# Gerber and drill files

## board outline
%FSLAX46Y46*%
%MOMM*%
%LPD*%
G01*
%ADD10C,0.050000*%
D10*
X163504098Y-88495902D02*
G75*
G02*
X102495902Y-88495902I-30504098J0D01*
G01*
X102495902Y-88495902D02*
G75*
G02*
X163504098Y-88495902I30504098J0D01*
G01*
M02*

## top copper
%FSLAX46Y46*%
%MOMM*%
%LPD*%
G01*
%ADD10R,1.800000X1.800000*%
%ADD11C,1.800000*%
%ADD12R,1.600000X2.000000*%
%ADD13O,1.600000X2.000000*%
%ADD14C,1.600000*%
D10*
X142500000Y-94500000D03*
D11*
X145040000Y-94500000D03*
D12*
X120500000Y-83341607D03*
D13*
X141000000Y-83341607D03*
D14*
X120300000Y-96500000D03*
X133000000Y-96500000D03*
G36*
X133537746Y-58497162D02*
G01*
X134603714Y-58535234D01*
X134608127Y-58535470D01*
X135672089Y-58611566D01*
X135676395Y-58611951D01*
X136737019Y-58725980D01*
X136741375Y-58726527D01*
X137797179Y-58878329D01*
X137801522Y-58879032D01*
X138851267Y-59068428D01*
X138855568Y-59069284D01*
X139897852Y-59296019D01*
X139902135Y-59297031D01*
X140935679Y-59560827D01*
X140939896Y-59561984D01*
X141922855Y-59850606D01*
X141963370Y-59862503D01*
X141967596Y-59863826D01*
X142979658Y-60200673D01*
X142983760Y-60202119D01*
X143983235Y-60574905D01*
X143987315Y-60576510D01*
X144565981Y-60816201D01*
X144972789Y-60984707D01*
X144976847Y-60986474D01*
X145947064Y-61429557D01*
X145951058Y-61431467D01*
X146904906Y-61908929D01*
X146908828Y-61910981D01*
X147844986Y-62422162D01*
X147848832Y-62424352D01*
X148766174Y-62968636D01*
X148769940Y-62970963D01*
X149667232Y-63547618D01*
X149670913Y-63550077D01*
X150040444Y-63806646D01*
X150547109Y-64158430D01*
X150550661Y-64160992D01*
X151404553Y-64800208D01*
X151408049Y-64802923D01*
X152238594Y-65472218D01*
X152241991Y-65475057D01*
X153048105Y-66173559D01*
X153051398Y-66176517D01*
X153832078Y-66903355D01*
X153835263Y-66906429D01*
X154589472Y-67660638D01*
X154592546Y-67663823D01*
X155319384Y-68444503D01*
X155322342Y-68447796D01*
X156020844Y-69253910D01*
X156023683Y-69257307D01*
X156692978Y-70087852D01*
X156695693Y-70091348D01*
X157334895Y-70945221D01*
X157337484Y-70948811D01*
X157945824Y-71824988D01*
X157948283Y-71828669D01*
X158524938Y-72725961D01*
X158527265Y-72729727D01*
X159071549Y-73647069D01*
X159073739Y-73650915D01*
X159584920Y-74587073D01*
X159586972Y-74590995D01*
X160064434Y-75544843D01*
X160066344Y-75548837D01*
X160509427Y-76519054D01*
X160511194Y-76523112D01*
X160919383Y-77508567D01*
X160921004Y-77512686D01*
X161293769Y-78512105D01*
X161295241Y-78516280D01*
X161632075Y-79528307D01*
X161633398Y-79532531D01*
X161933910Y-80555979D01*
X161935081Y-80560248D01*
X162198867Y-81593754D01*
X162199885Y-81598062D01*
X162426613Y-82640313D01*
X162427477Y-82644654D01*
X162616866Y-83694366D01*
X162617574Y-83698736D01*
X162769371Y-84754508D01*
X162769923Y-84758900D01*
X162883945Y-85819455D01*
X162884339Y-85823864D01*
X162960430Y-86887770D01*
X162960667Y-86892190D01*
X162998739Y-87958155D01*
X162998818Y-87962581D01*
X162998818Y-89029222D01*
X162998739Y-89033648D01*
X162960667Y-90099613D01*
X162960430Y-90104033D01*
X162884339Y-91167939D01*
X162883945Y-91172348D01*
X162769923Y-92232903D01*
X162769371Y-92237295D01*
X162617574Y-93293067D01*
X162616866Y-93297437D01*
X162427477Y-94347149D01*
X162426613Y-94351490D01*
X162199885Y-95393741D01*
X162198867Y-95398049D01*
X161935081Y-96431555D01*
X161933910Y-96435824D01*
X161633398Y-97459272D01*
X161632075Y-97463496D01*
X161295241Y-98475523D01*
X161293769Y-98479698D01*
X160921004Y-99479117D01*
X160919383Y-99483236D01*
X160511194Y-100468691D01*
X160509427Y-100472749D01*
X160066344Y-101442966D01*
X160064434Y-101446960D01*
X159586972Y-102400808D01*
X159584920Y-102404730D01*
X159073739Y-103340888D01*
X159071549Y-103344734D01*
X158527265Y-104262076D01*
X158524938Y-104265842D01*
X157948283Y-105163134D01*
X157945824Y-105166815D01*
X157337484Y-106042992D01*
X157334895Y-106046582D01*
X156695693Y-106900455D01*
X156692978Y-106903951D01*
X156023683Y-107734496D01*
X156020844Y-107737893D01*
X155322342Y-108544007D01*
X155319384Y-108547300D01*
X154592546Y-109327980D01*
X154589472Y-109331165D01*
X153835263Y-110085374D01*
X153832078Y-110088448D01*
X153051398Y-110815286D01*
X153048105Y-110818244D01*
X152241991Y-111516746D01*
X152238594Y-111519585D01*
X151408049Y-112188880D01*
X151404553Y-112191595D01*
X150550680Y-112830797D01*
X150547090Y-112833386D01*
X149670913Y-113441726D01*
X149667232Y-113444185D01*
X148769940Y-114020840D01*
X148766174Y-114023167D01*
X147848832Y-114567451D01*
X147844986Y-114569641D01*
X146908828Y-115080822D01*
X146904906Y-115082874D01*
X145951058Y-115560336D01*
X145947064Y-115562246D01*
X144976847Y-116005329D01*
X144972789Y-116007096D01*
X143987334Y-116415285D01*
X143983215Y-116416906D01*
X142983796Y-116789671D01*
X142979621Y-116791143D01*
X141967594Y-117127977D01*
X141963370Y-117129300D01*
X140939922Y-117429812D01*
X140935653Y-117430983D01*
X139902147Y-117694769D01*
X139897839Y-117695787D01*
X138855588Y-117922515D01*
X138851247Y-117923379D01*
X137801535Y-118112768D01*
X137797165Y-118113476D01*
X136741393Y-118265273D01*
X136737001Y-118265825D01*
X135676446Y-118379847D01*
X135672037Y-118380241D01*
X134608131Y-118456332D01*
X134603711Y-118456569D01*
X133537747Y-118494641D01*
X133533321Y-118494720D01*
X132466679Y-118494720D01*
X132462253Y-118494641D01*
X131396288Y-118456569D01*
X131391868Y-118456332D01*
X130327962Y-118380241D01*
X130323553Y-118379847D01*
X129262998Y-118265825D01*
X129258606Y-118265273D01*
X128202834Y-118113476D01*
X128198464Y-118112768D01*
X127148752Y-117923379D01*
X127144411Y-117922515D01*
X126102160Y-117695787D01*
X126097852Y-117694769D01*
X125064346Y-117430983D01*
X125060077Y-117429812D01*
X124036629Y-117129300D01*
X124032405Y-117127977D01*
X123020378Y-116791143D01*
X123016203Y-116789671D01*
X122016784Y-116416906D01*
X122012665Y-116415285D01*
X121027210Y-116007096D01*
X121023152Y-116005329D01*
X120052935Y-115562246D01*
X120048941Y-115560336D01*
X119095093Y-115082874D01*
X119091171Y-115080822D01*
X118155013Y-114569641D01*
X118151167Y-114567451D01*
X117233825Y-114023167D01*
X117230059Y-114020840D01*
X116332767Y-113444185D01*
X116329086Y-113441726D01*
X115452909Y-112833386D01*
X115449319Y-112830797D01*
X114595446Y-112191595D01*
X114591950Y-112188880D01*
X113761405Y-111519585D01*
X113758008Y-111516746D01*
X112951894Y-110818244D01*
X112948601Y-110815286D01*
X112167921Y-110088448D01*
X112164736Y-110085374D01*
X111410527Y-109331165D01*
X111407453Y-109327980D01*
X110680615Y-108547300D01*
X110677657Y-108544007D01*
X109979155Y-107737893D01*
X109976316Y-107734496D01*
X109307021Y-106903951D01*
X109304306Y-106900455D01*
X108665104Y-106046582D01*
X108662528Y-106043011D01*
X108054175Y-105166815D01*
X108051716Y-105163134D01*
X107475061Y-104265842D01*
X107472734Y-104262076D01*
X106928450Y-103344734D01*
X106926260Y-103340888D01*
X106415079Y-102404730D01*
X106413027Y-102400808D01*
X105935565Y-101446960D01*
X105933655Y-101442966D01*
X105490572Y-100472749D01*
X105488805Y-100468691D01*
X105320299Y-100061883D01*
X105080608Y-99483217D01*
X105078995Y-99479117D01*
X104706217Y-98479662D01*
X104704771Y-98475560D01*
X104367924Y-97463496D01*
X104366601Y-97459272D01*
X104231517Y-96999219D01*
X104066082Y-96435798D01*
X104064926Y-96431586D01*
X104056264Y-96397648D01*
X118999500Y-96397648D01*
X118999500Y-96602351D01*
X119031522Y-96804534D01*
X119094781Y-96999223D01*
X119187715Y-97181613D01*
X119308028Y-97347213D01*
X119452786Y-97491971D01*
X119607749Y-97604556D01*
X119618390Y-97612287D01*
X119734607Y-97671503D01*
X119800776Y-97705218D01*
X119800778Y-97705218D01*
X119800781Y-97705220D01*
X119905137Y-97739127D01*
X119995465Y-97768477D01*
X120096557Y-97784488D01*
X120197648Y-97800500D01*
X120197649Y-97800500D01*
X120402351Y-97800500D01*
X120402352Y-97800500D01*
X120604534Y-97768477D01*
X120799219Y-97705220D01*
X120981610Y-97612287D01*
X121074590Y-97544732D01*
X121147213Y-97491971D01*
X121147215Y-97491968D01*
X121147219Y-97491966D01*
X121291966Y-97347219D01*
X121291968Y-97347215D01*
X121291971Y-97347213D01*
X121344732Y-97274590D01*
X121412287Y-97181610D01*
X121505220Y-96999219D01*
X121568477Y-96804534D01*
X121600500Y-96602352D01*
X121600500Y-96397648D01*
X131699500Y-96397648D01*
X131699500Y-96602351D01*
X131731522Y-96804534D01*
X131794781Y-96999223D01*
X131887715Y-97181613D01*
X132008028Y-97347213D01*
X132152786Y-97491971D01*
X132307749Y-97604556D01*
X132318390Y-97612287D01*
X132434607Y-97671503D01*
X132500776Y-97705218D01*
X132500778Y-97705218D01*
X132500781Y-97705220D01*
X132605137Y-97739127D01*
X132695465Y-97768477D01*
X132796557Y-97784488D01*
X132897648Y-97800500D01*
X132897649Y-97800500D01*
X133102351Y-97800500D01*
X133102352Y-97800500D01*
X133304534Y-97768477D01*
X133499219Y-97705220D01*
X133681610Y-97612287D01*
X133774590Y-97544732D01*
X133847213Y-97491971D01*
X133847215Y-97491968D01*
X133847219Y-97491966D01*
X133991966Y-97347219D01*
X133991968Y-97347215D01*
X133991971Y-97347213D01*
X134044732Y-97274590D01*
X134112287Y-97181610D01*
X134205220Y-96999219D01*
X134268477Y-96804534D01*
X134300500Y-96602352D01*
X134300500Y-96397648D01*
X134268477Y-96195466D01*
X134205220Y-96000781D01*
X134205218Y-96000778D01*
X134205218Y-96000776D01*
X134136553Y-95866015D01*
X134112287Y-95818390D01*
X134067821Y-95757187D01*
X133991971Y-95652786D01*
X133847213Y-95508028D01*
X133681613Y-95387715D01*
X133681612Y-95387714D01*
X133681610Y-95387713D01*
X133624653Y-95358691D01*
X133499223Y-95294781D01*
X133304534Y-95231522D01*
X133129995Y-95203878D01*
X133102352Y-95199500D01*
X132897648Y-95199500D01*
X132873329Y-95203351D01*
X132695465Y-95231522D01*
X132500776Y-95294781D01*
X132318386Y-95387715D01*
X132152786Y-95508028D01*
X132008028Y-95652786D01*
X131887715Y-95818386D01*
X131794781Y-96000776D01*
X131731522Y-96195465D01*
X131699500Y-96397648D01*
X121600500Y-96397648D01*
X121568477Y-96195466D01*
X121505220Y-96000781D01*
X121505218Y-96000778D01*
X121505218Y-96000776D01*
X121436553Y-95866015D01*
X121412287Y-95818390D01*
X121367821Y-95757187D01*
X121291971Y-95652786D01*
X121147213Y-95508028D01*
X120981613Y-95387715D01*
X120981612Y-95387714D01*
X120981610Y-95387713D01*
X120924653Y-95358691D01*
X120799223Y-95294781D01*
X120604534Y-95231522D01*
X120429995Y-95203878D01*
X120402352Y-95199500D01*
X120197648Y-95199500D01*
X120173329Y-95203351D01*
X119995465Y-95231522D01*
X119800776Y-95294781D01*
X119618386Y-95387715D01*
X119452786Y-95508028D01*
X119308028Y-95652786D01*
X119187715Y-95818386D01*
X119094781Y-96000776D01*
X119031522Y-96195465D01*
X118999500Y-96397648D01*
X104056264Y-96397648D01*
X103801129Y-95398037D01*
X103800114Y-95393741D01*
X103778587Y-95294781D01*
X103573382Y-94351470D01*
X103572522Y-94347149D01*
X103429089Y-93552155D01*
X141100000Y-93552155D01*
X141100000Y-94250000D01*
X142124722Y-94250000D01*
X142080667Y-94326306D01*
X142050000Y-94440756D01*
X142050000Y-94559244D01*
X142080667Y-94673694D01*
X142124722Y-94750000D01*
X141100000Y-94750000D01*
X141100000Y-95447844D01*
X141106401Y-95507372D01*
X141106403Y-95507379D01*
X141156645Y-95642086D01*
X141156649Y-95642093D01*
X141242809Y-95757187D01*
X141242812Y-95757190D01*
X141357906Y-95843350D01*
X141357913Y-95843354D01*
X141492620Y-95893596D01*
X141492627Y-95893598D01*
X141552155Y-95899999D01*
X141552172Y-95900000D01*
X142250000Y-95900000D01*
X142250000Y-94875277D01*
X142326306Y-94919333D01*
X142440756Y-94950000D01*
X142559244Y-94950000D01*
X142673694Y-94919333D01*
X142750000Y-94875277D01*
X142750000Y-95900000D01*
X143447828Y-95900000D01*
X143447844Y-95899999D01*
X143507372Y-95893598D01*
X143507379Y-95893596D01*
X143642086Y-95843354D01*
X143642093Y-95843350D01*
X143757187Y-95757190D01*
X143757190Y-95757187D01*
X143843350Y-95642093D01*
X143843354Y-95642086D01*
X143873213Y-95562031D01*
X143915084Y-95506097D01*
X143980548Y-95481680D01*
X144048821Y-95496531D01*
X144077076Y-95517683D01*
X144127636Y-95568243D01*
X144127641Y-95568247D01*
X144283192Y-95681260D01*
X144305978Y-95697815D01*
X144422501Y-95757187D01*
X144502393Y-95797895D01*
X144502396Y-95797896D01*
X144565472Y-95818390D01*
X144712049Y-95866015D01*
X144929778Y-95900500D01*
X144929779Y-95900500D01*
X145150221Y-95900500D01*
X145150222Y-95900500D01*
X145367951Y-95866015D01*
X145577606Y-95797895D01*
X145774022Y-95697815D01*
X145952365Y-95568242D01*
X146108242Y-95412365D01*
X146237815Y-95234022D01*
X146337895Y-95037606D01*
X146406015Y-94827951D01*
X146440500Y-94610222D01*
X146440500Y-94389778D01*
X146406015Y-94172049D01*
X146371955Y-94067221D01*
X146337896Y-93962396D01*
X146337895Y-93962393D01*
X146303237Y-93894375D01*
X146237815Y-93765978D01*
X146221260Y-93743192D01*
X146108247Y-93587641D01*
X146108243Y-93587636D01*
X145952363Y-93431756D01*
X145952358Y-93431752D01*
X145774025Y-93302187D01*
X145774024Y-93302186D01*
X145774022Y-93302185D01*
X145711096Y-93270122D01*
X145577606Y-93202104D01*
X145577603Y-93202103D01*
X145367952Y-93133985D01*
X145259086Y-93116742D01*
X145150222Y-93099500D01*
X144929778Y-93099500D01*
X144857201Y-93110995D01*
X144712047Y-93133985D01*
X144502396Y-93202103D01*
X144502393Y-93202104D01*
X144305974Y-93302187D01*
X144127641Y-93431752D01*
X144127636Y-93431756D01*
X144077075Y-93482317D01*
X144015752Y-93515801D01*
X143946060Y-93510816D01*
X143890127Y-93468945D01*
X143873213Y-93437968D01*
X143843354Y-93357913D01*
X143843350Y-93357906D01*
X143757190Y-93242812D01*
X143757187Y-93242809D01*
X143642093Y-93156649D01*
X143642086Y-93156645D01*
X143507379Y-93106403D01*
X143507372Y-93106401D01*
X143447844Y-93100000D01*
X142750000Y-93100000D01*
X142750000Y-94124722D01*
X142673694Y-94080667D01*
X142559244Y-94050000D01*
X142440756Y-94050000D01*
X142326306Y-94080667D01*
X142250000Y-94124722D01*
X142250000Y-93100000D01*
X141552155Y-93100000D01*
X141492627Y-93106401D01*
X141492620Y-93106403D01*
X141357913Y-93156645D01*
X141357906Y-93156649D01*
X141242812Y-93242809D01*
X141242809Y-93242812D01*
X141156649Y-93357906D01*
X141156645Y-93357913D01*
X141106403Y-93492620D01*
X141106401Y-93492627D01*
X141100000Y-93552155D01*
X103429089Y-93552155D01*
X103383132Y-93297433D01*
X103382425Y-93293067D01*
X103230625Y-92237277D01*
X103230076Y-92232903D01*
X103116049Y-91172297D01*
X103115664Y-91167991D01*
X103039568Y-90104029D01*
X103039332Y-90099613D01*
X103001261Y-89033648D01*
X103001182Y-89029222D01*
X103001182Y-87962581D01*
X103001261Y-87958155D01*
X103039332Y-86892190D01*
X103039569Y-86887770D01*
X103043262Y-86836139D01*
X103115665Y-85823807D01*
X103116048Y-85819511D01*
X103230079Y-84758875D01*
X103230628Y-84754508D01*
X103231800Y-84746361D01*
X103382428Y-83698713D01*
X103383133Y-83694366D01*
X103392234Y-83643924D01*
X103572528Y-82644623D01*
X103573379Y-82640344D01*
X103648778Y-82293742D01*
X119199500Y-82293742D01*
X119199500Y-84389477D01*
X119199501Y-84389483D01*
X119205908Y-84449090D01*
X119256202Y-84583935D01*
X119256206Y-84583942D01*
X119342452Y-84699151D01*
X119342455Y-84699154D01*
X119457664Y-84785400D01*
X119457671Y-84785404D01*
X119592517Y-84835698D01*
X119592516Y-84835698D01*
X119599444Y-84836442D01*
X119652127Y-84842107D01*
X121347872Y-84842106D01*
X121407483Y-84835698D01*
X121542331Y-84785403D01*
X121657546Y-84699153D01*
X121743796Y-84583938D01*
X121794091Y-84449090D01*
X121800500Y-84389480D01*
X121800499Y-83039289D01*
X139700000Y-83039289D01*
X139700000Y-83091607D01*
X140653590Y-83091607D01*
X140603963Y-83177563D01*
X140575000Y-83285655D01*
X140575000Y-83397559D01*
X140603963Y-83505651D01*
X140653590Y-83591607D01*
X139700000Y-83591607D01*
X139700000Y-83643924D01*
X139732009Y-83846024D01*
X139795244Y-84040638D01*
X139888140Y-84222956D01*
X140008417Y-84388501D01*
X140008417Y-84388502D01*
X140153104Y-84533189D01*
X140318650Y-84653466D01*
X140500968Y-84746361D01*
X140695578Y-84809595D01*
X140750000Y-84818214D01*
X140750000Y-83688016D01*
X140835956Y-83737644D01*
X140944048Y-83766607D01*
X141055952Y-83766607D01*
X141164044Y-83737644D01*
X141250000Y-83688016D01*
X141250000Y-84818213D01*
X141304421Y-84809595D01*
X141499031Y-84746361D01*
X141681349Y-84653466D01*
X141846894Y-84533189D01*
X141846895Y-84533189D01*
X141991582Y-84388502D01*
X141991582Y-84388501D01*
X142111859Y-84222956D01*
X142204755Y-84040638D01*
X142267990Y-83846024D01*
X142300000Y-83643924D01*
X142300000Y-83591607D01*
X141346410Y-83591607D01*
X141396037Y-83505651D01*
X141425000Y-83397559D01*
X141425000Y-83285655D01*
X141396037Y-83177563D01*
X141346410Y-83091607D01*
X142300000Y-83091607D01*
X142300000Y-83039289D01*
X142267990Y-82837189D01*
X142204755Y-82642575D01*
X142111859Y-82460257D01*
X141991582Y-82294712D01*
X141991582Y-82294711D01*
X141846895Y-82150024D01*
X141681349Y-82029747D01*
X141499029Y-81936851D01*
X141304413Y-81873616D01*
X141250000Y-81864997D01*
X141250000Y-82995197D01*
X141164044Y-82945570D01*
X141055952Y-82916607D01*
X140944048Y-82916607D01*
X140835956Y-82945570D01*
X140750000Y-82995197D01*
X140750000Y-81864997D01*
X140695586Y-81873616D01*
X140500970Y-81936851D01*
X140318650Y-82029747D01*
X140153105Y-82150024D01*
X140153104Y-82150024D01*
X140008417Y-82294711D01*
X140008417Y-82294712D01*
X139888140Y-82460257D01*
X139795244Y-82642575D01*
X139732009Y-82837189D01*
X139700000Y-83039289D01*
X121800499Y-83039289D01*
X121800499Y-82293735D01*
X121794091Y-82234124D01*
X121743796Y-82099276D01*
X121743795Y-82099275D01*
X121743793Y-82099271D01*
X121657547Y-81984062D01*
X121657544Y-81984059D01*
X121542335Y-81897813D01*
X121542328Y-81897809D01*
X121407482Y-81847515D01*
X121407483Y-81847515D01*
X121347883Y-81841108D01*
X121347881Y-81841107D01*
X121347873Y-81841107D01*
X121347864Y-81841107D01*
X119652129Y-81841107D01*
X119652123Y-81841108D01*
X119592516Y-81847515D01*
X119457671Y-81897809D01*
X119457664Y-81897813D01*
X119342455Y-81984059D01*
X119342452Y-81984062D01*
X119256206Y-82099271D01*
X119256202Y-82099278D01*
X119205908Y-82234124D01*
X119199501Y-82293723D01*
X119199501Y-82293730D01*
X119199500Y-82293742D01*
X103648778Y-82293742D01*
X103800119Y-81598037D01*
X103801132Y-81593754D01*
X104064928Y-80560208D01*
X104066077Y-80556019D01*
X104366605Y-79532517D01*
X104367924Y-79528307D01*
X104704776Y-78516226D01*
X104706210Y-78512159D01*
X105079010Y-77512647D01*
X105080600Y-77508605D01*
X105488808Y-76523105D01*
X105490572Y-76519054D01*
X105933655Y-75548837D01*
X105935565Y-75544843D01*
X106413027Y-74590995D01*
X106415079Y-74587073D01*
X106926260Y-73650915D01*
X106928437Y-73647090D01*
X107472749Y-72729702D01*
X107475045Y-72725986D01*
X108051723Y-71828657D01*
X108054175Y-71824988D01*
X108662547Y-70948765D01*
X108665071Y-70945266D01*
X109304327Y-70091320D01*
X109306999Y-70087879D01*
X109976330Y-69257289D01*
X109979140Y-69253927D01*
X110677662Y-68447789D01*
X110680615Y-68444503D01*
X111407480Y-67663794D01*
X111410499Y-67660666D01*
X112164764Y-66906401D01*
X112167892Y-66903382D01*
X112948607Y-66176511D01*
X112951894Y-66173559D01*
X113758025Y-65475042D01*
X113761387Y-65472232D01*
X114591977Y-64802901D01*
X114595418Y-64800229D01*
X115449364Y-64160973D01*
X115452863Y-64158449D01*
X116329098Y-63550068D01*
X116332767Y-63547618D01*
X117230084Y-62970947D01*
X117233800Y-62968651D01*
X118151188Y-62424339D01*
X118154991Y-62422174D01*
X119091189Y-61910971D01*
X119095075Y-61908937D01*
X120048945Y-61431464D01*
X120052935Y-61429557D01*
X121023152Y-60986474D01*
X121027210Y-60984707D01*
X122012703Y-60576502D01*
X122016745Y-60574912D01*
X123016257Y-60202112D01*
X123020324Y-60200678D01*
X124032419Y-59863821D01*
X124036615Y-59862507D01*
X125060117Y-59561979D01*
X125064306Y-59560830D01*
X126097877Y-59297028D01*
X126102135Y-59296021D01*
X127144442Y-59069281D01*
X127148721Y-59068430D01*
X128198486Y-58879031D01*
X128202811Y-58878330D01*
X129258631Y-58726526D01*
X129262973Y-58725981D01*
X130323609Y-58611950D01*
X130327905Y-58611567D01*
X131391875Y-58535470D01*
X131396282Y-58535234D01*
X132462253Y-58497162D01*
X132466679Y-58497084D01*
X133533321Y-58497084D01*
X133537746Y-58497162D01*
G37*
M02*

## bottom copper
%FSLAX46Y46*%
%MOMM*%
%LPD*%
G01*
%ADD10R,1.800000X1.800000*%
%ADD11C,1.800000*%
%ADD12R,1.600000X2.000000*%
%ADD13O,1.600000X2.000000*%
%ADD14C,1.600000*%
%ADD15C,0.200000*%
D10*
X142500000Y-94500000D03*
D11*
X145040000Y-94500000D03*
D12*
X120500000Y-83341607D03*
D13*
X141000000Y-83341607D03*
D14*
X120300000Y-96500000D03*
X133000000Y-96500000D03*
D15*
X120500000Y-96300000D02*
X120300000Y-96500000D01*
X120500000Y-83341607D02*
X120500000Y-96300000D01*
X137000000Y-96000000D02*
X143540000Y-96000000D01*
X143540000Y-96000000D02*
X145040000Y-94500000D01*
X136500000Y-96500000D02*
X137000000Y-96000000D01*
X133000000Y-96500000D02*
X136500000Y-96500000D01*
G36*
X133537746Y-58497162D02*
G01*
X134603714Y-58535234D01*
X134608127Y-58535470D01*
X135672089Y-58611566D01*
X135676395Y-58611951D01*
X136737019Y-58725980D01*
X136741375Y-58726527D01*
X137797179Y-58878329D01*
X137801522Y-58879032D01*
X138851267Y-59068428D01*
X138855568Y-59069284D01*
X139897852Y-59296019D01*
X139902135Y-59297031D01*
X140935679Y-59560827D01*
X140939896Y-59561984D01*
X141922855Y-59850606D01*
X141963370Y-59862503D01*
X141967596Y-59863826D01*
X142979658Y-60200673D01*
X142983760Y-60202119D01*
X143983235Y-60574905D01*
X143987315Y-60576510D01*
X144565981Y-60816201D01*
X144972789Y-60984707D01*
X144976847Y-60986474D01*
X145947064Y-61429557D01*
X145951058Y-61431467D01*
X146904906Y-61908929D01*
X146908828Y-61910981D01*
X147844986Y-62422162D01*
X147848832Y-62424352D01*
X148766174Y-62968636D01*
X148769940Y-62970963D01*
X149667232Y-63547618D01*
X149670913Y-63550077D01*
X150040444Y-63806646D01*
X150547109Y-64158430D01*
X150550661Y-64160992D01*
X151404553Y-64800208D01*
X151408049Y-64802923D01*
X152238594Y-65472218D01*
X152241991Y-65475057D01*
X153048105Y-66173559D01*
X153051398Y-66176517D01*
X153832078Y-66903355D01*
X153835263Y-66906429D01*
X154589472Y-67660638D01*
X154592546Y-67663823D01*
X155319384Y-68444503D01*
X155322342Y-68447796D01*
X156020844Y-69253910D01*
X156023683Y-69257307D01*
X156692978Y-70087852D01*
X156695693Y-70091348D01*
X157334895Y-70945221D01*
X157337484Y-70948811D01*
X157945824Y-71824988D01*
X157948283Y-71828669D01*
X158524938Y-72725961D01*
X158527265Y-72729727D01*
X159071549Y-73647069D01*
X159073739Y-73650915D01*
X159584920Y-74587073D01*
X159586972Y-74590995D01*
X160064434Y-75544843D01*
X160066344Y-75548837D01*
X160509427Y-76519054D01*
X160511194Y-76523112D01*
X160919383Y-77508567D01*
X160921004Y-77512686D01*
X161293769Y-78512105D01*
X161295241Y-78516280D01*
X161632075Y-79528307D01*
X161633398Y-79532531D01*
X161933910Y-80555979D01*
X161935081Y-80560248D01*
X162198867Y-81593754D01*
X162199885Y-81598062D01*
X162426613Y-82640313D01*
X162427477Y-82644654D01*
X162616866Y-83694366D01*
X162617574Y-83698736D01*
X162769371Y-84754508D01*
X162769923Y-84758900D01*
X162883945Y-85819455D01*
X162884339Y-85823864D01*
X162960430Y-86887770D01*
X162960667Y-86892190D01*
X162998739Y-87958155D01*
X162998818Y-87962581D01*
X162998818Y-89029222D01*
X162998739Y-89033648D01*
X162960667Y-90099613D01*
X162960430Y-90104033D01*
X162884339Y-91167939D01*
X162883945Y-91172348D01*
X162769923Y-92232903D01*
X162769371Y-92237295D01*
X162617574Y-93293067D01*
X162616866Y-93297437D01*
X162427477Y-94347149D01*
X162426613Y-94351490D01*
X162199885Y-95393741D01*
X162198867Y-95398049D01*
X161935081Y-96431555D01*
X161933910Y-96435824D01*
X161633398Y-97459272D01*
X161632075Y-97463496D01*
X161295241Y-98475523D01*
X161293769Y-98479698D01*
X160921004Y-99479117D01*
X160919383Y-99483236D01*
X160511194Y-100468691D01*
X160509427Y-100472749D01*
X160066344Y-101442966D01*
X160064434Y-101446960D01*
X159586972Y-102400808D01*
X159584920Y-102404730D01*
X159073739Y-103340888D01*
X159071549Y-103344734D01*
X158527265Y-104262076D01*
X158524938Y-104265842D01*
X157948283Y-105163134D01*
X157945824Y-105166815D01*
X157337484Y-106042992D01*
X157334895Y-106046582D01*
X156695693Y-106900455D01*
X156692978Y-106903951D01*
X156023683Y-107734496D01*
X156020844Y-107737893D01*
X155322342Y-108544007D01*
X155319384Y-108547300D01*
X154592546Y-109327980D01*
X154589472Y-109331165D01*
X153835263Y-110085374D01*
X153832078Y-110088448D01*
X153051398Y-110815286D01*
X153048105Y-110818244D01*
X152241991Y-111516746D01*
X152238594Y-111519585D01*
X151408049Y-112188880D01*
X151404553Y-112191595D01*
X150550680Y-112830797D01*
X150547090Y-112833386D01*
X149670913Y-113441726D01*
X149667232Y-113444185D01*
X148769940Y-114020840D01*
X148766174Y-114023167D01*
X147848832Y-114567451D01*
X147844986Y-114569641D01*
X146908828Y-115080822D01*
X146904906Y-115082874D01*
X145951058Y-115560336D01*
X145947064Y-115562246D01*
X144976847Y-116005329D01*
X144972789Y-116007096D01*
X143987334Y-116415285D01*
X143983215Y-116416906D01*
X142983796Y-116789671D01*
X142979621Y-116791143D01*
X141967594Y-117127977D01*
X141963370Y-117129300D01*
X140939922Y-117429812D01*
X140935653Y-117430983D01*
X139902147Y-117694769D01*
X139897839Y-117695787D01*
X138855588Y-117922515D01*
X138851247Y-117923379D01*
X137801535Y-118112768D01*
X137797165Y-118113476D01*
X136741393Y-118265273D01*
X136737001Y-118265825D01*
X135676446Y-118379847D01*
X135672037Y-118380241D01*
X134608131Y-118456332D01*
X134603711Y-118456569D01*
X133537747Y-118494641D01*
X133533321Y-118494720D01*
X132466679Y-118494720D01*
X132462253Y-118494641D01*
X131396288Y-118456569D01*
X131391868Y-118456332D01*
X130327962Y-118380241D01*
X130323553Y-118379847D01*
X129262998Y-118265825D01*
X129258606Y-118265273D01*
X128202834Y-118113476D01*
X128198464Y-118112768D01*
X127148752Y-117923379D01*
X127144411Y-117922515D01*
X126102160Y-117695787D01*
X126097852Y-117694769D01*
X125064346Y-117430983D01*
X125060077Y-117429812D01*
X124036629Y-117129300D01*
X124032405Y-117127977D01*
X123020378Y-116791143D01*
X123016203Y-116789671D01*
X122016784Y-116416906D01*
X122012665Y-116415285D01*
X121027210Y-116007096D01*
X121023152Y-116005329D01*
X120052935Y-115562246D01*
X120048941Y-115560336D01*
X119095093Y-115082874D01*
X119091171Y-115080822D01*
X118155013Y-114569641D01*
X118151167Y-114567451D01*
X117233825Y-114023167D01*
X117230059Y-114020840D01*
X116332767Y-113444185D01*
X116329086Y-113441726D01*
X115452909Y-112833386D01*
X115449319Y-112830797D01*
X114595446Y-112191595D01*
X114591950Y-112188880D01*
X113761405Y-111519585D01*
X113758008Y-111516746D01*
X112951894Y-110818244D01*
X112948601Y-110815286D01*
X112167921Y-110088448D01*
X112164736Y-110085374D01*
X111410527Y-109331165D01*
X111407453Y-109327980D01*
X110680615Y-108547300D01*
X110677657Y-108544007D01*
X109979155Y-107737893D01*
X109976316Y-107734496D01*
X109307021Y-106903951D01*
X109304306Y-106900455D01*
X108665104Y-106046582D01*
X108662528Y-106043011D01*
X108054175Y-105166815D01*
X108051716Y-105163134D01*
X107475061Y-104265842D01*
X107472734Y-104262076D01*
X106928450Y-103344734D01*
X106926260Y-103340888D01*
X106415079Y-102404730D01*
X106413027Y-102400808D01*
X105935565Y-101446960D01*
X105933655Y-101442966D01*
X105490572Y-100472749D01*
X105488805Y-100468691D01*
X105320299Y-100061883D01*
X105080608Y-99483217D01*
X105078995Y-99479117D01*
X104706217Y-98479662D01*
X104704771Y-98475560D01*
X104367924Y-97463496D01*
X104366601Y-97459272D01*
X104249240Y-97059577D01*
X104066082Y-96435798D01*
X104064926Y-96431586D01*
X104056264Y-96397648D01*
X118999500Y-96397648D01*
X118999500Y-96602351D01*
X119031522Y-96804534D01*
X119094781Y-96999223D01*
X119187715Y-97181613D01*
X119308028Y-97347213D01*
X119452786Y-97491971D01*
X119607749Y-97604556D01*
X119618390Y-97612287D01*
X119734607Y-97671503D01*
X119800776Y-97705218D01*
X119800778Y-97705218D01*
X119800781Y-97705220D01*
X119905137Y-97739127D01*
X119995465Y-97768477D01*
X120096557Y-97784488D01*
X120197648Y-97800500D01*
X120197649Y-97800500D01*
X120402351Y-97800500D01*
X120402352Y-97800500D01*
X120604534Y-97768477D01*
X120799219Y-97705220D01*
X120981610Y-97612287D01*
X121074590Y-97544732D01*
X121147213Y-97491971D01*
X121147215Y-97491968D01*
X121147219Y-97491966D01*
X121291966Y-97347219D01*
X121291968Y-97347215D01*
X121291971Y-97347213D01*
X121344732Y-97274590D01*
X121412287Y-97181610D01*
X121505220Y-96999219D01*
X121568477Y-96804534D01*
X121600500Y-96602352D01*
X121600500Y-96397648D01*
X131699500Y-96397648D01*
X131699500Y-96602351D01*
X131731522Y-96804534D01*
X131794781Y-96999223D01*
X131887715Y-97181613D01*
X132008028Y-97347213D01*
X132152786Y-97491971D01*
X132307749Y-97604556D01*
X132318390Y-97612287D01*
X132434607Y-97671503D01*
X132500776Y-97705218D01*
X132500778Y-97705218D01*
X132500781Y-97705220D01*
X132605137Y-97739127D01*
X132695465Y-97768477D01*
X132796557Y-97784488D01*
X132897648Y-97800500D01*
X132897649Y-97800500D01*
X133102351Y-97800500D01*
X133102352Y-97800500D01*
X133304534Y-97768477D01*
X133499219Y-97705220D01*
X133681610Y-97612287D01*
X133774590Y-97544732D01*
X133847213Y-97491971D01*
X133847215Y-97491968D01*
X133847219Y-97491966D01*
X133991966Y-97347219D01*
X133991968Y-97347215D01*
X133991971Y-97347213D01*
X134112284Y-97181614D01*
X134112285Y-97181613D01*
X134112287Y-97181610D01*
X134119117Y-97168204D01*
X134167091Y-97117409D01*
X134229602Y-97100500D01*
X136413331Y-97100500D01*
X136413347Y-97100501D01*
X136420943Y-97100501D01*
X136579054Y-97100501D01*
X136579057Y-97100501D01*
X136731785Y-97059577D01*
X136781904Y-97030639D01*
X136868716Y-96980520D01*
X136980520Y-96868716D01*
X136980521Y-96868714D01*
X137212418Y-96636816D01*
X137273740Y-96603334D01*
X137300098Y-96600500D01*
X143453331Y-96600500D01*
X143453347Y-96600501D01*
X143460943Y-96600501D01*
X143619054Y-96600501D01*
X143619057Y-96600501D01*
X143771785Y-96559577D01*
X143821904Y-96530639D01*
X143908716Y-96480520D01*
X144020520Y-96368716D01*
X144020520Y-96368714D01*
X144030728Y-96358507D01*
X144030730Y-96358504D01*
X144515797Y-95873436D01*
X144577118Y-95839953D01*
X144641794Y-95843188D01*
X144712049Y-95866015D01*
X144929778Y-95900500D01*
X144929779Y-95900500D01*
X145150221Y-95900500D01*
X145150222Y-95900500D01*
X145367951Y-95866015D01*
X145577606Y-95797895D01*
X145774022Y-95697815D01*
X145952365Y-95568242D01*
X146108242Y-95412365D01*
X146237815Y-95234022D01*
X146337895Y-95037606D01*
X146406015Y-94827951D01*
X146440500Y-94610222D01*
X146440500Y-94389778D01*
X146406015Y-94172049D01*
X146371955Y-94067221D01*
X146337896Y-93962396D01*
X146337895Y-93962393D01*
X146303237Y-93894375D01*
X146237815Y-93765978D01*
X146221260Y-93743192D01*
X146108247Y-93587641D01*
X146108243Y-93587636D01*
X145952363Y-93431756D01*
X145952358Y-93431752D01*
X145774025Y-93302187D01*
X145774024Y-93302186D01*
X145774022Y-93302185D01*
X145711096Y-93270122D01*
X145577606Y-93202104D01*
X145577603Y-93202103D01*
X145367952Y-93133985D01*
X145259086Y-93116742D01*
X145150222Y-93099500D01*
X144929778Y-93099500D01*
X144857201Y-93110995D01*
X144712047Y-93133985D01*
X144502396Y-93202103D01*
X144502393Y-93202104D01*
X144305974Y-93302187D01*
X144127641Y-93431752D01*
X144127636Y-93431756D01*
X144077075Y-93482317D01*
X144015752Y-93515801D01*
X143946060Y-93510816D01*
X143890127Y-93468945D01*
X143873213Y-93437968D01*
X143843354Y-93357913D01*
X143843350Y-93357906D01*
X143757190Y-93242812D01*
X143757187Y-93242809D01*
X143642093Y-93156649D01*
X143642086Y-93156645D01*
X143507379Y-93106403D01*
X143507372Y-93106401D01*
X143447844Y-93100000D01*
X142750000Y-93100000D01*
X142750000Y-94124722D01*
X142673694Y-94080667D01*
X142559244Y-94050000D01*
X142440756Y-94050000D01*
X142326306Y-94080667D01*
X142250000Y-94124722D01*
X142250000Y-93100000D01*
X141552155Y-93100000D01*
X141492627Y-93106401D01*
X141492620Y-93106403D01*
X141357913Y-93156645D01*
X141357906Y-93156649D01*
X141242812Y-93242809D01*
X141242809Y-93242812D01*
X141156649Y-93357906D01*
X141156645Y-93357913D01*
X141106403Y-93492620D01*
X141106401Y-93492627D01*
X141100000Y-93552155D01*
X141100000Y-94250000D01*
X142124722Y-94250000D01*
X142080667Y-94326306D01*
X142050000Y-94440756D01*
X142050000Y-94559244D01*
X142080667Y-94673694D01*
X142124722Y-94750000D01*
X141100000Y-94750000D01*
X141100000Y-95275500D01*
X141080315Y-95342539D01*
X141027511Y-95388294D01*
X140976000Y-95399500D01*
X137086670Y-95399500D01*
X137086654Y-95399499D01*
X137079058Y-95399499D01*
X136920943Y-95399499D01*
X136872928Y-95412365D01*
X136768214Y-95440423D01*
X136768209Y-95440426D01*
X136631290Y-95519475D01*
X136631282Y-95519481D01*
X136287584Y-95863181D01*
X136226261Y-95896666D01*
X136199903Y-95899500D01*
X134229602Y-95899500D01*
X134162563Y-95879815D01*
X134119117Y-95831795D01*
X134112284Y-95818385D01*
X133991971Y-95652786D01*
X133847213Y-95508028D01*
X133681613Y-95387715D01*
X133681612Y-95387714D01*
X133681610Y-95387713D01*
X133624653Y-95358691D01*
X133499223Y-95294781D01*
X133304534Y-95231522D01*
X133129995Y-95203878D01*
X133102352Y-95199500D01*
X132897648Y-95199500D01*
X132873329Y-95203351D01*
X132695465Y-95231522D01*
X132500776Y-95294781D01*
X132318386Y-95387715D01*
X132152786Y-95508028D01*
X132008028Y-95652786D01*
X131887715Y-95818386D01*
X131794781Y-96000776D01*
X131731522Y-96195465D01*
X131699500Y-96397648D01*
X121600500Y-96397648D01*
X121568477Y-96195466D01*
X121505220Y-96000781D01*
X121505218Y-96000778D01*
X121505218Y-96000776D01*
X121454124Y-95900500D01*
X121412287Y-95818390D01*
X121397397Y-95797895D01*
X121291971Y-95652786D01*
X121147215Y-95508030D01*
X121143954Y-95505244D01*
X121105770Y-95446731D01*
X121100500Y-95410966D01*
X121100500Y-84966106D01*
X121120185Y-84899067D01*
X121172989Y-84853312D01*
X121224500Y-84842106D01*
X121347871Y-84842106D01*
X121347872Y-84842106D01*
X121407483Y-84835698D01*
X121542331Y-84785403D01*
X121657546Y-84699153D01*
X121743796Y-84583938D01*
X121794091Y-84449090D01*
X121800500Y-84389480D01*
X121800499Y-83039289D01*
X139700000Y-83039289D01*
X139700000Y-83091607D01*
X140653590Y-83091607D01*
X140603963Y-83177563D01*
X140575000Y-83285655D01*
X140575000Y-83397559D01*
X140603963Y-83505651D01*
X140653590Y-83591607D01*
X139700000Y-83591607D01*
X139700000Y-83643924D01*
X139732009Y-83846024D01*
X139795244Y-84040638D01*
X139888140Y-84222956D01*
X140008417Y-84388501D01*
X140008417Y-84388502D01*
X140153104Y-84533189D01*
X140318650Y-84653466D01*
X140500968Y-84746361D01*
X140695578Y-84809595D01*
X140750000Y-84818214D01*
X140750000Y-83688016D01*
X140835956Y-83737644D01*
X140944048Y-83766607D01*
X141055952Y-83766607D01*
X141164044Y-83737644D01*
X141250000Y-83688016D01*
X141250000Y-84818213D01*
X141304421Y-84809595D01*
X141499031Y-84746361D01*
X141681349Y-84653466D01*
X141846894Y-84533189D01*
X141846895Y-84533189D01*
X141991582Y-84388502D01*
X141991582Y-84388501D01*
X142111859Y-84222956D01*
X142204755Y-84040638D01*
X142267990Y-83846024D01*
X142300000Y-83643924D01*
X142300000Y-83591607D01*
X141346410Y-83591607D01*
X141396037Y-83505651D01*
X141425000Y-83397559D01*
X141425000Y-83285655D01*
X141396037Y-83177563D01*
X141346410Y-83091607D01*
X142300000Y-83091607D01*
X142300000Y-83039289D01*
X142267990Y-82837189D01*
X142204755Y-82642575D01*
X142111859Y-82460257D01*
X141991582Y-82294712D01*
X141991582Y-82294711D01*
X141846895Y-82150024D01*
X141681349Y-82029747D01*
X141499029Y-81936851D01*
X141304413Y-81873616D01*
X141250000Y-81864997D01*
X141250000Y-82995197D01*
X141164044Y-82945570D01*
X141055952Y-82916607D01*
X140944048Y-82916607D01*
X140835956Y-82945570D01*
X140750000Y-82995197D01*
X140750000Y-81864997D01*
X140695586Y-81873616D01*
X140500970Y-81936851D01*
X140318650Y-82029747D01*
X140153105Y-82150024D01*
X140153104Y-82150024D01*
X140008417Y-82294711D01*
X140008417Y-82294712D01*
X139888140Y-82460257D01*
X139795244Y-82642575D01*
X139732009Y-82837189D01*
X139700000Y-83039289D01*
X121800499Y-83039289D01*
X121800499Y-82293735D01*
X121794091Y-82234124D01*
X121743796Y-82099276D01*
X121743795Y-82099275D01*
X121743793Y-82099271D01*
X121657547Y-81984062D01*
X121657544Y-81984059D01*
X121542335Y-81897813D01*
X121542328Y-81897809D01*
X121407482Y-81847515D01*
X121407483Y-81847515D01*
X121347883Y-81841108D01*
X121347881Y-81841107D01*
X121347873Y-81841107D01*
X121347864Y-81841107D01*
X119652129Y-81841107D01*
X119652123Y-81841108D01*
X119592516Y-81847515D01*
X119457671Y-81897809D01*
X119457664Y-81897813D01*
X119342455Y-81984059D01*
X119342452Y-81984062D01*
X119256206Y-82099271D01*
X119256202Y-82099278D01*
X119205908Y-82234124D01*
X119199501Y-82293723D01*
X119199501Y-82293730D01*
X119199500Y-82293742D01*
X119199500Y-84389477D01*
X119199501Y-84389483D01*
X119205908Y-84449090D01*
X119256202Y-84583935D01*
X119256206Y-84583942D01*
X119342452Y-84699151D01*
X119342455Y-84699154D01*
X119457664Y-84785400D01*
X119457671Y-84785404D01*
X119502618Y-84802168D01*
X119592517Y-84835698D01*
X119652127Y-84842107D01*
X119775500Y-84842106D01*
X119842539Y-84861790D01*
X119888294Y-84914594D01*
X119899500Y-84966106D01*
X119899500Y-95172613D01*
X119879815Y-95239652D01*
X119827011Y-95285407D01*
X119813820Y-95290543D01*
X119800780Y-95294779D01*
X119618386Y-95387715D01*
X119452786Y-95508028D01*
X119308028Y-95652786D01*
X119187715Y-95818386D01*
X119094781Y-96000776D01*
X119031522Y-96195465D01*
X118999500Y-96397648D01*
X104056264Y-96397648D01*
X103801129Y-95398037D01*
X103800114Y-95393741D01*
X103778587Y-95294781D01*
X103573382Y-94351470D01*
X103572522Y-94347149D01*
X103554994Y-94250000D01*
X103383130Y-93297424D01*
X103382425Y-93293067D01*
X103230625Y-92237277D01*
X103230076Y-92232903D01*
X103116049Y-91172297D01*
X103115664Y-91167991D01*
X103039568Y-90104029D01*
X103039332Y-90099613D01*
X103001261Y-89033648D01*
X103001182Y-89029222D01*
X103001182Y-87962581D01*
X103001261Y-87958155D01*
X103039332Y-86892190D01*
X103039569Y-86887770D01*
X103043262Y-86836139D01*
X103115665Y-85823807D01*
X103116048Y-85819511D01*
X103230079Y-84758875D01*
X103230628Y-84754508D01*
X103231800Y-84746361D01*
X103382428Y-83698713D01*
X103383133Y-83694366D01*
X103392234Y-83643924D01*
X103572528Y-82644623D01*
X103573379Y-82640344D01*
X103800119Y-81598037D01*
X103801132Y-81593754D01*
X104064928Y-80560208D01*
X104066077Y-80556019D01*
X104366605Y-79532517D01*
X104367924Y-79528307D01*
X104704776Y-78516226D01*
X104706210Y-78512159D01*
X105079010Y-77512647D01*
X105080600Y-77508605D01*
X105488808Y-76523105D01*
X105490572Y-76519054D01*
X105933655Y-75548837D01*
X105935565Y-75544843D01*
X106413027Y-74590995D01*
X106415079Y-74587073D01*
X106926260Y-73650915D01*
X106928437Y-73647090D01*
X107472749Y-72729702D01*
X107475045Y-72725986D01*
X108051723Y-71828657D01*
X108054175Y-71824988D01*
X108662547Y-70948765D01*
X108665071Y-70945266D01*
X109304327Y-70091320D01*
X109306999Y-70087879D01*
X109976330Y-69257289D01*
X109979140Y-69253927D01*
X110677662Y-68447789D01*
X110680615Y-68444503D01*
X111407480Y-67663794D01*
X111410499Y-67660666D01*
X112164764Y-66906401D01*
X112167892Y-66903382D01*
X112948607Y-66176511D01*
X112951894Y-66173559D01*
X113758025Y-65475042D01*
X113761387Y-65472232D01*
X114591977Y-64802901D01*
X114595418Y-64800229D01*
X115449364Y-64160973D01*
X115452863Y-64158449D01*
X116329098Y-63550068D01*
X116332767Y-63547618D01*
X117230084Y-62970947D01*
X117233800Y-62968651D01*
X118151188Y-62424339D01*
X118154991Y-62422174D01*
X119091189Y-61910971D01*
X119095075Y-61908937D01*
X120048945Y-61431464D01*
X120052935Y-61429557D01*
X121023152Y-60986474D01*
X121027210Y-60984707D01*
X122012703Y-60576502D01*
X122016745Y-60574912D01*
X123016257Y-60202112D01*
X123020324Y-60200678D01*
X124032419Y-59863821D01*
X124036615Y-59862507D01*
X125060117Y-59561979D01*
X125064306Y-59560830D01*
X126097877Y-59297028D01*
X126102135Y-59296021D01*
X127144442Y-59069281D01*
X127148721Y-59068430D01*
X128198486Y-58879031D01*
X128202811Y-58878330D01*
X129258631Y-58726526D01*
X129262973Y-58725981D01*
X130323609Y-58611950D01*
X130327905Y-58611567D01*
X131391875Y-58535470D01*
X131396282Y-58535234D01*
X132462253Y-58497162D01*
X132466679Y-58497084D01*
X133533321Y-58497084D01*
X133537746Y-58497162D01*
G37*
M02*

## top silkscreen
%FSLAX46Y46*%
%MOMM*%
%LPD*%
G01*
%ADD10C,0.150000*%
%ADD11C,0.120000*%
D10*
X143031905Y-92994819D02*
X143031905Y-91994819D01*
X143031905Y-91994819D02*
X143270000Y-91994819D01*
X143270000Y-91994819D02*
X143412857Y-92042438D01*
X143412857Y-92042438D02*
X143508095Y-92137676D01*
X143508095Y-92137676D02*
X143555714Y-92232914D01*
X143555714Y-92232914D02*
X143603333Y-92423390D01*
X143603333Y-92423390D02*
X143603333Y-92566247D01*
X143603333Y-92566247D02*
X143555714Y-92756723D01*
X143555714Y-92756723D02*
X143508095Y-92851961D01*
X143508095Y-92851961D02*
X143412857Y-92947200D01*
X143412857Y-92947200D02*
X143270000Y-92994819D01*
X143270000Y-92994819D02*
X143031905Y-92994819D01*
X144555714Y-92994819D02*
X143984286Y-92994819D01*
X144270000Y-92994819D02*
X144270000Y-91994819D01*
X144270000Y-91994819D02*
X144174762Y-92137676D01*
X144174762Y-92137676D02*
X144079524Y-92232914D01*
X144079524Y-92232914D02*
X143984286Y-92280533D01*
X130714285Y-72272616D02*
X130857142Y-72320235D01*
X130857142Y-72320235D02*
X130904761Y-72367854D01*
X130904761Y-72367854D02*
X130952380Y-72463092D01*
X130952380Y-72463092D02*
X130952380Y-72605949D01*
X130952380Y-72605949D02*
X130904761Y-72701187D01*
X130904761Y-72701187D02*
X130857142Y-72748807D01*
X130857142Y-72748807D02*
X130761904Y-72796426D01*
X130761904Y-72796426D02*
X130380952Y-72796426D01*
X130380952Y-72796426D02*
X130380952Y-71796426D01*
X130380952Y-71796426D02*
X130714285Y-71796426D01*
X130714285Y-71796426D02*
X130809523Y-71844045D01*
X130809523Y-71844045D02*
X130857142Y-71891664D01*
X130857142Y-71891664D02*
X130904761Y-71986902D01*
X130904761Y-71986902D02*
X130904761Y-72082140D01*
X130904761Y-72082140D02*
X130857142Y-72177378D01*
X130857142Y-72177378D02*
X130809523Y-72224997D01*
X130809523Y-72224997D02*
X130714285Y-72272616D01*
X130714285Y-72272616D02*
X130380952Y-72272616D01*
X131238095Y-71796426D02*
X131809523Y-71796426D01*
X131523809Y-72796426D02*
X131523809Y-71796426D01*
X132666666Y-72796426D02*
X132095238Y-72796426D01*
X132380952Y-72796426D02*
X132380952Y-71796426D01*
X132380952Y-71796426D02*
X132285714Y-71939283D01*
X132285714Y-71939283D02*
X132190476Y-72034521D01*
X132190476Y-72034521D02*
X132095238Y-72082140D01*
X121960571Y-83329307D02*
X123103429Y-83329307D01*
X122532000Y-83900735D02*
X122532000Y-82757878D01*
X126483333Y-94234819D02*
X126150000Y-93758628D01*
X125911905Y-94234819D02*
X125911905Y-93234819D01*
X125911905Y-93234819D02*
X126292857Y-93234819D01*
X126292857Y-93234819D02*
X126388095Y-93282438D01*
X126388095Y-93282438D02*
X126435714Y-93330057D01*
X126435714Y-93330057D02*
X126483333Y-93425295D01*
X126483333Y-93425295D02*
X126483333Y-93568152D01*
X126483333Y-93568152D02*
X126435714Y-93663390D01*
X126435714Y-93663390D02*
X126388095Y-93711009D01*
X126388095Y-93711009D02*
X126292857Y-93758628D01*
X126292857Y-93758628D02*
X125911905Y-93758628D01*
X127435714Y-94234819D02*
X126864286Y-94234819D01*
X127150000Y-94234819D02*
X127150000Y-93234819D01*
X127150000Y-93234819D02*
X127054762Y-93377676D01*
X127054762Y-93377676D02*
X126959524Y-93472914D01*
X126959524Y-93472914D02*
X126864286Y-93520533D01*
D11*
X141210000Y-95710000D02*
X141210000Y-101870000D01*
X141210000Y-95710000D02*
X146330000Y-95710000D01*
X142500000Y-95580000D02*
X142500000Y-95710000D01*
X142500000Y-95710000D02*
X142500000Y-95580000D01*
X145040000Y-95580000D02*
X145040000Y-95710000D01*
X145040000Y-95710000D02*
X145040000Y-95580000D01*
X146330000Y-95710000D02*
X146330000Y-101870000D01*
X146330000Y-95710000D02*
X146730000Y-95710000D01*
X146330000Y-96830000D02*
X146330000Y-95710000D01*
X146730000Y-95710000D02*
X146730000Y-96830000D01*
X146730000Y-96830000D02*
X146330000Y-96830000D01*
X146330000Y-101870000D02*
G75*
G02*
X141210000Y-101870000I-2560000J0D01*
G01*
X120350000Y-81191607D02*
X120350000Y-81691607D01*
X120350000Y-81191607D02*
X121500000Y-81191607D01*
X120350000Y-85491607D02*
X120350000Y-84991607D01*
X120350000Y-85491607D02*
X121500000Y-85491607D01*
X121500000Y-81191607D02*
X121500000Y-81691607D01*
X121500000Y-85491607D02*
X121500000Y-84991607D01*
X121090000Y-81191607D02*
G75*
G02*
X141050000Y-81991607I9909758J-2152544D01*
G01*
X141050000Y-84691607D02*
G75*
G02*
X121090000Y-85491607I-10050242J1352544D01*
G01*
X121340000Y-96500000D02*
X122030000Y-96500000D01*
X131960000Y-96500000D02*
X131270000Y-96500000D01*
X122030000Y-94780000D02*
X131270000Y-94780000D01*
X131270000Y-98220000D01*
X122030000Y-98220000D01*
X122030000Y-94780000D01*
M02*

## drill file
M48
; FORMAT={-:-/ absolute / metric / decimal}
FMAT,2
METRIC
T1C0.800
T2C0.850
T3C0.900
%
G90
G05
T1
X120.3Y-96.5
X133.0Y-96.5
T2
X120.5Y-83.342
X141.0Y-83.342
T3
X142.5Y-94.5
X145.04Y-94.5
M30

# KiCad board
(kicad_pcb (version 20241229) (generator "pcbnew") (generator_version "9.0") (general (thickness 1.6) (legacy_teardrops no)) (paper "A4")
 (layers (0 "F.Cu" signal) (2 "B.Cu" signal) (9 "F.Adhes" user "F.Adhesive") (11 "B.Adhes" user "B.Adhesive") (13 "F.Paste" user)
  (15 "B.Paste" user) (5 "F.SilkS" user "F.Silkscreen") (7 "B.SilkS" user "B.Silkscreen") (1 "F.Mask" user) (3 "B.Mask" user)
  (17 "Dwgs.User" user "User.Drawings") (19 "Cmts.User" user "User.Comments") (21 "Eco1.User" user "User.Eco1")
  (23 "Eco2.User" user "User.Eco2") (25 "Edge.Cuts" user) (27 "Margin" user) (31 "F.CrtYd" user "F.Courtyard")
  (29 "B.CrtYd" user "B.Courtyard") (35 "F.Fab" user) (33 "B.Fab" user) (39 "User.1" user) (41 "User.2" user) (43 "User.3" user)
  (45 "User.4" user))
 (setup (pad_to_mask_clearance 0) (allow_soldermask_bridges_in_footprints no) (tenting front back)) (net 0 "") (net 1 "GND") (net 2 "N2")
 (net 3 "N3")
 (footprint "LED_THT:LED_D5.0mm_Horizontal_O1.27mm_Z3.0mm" (layer "F.Cu") (at 142.5 94.5)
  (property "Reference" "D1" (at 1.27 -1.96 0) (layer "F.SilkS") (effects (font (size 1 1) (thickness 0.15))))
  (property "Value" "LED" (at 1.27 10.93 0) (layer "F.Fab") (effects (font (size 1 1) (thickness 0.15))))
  (fp_line (start -1.29 1.21) (end -1.29 7.37) (stroke (width 0.12) (type solid)) (layer "F.SilkS"))
  (fp_line (start -1.29 1.21) (end 3.83 1.21) (stroke (width 0.12) (type solid)) (layer "F.SilkS"))
  (fp_line (start 0 1.08) (end 0 1.21) (stroke (width 0.12) (type solid)) (layer "F.SilkS"))
  (fp_line (start 0 1.21) (end 0 1.08) (stroke (width 0.12) (type solid)) (layer "F.SilkS"))
  (fp_line (start 2.54 1.08) (end 2.54 1.21) (stroke (width 0.12) (type solid)) (layer "F.SilkS"))
  (fp_line (start 2.54 1.21) (end 2.54 1.08) (stroke (width 0.12) (type solid)) (layer "F.SilkS"))
  (fp_line (start 3.83 1.21) (end 3.83 7.37) (stroke (width 0.12) (type solid)) (layer "F.SilkS"))
  (fp_line (start 3.83 1.21) (end 4.23 1.21) (stroke (width 0.12) (type solid)) (layer "F.SilkS"))
  (fp_line (start 3.83 2.33) (end 3.83 1.21) (stroke (width 0.12) (type solid)) (layer "F.SilkS"))
  (fp_line (start 4.23 1.21) (end 4.23 2.33) (stroke (width 0.12) (type solid)) (layer "F.SilkS"))
  (fp_line (start 4.23 2.33) (end 3.83 2.33) (stroke (width 0.12) (type solid)) (layer "F.SilkS"))
  (fp_arc (start 3.83 7.37) (mid 1.27 9.93) (end -1.29 7.37) (stroke (width 0.12) (type solid)) (layer "F.SilkS"))
  (pad "1" thru_hole rect (at 0 0) (size 1.8 1.8) (drill 0.9) (layers "*.Cu" "*.Mask") (remove_unused_layers no) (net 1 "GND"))
  (pad "2" thru_hole circle (at 2.54 0) (size 1.8 1.8) (drill 0.9) (layers "*.Cu" "*.Mask") (remove_unused_layers no) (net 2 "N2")))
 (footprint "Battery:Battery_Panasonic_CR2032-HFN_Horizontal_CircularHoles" (layer "F.Cu") (at 120.5 83.341607)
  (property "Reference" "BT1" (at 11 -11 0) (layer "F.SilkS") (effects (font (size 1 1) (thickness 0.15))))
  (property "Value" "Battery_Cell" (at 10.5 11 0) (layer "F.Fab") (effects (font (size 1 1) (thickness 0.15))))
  (fp_line (start -0.15 -2.15) (end -0.15 -1.65) (stroke (width 0.12) (type default)) (layer "F.SilkS"))
  (fp_line (start -0.15 -2.15) (end 1 -2.15) (stroke (width 0.12) (type default)) (layer "F.SilkS"))
  (fp_line (start -0.15 2.15) (end -0.15 1.65) (stroke (width 0.12) (type default)) (layer "F.SilkS"))
  (fp_line (start -0.15 2.15) (end 1 2.15) (stroke (width 0.12) (type default)) (layer "F.SilkS"))
  (fp_line (start 1 -2.15) (end 1 -1.65) (stroke (width 0.12) (type default)) (layer "F.SilkS"))
  (fp_line (start 1 2.15) (end 1 1.65) (stroke (width 0.12) (type default)) (layer "F.SilkS"))
  (fp_arc (start 0.59 -2.15) (mid 10.91 -10.13) (end 20.55 -1.35) (stroke (width 0.12) (type default)) (layer "F.SilkS"))
  (fp_arc (start 20.55 1.35) (mid 10.91 10.13) (end 0.59 2.15) (stroke (width 0.12) (type default)) (layer "F.SilkS"))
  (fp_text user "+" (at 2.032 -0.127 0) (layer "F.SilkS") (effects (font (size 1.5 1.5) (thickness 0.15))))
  (pad "1" thru_hole rect (at 0 0) (size 1.6 2) (drill 0.85) (layers "*.Cu" "*.Mask") (remove_unused_layers no) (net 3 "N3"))
  (pad "2" thru_hole oval (at 20.5 0) (size 1.6 2) (drill 0.85) (layers "*.Cu" "*.Mask") (remove_unused_layers no) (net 1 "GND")))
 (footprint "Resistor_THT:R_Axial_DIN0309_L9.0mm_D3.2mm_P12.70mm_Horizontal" (layer "F.Cu") (at 120.3 96.5)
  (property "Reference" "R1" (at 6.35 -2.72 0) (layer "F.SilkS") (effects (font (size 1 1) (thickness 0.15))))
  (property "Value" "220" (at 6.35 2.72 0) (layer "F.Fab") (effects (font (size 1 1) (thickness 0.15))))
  (fp_line (start 1.04 0) (end 1.73 0) (stroke (width 0.12) (type solid)) (layer "F.SilkS"))
  (fp_line (start 11.66 0) (end 10.97 0) (stroke (width 0.12) (type solid)) (layer "F.SilkS"))
  (fp_rect (start 1.73 -1.72) (end 10.97 1.72) (stroke (width 0.12) (type solid)) (fill no) (layer "F.SilkS"))
  (pad "1" thru_hole circle (at 0 0) (size 1.6 1.6) (drill 0.8) (layers "*.Cu" "*.Mask") (remove_unused_layers no) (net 3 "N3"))
  (pad "2" thru_hole circle (at 12.7 0) (size 1.6 1.6) (drill 0.8) (layers "*.Cu" "*.Mask") (remove_unused_layers no) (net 2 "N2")))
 (gr_circle (center 133 88.495902) (end 102.5 87.995902) (stroke (width 0.05) (type default)) (fill no) (layer "Edge.Cuts"))
 (segment (start 120.5 96.3) (end 120.3 96.5) (width 0.2) (layer "B.Cu") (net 3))
 (segment (start 120.5 83.341607) (end 120.5 96.3) (width 0.2) (layer "B.Cu") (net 3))
 (segment (start 137 96) (end 143.54 96) (width 0.2) (layer "B.Cu") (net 2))
 (segment (start 143.54 96) (end 145.04 94.5) (width 0.2) (layer "B.Cu") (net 2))
 (segment (start 136.5 96.5) (end 137 96) (width 0.2) (layer "B.Cu") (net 2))
 (segment (start 133 96.5) (end 136.5 96.5) (width 0.2) (layer "B.Cu") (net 2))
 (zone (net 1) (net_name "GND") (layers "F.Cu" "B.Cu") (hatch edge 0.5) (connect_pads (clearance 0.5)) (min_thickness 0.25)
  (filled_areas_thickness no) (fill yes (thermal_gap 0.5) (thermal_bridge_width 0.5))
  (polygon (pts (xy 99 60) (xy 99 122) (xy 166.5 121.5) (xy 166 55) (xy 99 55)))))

